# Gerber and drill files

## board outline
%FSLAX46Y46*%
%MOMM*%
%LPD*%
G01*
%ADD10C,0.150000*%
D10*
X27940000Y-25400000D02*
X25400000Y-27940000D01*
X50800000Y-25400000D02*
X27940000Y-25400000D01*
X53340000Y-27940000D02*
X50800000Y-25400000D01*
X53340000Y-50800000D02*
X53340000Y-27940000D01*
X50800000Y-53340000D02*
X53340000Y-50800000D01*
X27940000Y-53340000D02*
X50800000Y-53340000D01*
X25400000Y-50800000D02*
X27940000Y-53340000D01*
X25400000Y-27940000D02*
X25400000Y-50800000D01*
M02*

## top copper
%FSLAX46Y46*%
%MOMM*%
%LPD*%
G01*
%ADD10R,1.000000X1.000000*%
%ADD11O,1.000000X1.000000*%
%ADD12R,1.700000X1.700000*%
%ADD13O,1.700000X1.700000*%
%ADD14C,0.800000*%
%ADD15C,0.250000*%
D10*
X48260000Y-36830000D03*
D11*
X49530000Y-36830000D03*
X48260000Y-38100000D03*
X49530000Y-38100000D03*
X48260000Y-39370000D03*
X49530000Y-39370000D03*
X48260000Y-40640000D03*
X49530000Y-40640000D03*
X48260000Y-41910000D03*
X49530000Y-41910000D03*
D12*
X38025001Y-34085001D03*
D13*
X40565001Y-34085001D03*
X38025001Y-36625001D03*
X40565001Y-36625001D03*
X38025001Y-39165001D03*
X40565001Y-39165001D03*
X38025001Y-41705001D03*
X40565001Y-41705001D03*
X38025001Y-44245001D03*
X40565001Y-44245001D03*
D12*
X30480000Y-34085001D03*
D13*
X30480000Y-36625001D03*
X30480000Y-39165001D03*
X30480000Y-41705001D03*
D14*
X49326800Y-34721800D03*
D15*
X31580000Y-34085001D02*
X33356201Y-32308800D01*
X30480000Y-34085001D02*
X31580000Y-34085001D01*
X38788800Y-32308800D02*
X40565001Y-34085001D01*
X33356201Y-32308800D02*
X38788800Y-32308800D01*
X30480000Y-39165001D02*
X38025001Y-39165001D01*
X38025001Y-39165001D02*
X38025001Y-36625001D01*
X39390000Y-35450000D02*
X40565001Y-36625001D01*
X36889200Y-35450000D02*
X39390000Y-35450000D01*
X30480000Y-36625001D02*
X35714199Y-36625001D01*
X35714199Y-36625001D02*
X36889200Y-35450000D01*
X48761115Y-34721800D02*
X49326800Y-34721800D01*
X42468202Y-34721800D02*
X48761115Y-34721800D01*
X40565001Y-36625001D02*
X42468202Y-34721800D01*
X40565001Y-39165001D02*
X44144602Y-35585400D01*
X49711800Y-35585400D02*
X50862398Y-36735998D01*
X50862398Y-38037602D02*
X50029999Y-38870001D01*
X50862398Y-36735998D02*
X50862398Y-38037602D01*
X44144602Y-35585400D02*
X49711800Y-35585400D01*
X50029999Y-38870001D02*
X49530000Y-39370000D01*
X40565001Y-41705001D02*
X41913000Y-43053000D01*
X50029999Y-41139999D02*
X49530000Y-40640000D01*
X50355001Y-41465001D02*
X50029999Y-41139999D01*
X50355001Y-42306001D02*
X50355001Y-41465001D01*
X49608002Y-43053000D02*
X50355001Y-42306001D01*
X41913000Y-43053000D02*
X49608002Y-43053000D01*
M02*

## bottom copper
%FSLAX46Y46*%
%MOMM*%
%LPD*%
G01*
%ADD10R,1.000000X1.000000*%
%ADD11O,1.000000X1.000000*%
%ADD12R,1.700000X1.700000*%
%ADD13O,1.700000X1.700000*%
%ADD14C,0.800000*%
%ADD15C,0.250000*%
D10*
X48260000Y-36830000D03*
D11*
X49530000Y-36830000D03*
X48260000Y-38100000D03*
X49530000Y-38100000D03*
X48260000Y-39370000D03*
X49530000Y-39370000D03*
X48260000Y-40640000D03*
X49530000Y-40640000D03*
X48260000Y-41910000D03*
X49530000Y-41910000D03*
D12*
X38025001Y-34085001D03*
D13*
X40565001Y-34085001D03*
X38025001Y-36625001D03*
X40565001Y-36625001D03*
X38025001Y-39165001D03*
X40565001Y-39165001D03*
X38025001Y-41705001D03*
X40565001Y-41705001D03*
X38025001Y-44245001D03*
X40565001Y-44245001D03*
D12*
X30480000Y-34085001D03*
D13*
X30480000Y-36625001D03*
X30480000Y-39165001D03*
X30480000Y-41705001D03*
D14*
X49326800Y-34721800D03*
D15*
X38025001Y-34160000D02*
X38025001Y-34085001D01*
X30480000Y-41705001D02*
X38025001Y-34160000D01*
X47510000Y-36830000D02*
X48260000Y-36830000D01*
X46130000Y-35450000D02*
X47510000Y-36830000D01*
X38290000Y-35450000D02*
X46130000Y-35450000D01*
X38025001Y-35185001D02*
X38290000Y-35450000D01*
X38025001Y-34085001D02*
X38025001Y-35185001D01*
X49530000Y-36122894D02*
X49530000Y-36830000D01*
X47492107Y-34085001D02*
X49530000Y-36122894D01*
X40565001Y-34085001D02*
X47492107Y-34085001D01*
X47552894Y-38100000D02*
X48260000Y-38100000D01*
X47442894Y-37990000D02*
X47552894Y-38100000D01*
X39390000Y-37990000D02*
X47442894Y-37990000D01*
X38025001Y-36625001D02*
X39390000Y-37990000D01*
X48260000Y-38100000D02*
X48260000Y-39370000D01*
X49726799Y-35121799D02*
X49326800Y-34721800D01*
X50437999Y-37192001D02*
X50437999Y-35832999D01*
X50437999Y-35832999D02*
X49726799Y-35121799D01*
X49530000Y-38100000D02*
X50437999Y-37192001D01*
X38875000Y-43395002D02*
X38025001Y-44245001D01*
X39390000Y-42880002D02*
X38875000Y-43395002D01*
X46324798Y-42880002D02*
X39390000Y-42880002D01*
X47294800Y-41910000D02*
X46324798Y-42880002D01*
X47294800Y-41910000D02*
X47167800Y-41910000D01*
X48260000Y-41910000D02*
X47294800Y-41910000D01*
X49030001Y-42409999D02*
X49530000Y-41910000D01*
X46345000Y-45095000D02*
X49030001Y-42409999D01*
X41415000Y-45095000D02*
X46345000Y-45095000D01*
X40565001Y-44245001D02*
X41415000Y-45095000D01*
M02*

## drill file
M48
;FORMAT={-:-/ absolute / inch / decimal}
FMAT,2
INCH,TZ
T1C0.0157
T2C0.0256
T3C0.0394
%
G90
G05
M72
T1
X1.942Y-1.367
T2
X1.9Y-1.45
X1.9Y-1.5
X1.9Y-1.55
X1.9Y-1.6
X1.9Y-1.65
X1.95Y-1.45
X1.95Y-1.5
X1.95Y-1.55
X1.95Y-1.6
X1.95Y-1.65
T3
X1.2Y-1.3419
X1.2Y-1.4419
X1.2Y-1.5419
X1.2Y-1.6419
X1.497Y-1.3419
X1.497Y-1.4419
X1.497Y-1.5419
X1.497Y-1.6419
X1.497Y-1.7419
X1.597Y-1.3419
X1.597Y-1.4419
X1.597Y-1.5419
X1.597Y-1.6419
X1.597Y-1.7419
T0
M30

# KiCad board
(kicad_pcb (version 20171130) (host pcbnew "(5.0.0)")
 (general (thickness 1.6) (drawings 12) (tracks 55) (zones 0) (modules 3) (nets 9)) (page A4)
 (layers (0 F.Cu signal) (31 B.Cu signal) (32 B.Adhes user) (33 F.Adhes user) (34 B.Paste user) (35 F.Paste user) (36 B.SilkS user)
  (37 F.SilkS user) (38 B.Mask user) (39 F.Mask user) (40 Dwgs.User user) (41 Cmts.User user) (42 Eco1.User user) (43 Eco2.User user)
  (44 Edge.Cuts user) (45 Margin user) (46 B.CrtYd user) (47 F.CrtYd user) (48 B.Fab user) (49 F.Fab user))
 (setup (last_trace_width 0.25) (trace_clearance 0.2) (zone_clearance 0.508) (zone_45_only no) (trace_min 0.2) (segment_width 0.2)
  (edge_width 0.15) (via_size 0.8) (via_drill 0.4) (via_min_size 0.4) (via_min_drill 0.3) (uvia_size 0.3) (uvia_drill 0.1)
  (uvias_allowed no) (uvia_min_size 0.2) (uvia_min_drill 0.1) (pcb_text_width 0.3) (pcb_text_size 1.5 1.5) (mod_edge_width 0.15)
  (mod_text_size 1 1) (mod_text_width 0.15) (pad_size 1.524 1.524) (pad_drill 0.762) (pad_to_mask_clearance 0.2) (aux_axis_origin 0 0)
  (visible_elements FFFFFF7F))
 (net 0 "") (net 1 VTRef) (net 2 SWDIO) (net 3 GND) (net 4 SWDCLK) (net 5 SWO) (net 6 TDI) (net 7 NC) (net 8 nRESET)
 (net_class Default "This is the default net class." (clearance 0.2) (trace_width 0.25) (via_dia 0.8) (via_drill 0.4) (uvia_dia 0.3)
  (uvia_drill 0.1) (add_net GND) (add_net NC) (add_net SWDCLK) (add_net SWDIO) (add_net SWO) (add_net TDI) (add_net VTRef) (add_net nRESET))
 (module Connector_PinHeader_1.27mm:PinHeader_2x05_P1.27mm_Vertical (layer F.Cu) (at 48.26 36.83)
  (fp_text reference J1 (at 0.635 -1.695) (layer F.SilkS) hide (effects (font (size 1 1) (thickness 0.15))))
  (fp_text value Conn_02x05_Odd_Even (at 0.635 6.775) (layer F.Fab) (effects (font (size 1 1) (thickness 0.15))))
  (pad 1 thru_hole rect (at 0 0) (size 1 1) (drill 0.65) (layers *.Cu *.Mask) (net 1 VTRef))
  (pad 2 thru_hole oval (at 1.27 0) (size 1 1) (drill 0.65) (layers *.Cu *.Mask) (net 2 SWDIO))
  (pad 3 thru_hole oval (at 0 1.27) (size 1 1) (drill 0.65) (layers *.Cu *.Mask) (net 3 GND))
  (pad 4 thru_hole oval (at 1.27 1.27) (size 1 1) (drill 0.65) (layers *.Cu *.Mask) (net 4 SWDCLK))
  (pad 5 thru_hole oval (at 0 2.54) (size 1 1) (drill 0.65) (layers *.Cu *.Mask) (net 3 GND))
  (pad 6 thru_hole oval (at 1.27 2.54) (size 1 1) (drill 0.65) (layers *.Cu *.Mask) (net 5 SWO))
  (pad 7 thru_hole oval (at 0 3.81) (size 1 1) (drill 0.65) (layers *.Cu *.Mask))
  (pad 8 thru_hole oval (at 1.27 3.81) (size 1 1) (drill 0.65) (layers *.Cu *.Mask) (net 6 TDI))
  (pad 9 thru_hole oval (at 0 5.08) (size 1 1) (drill 0.65) (layers *.Cu *.Mask) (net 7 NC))
  (pad 10 thru_hole oval (at 1.27 5.08) (size 1 1) (drill 0.65) (layers *.Cu *.Mask) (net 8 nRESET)))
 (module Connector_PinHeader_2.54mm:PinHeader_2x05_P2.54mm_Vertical (layer F.Cu) (at 38.025001 34.085001)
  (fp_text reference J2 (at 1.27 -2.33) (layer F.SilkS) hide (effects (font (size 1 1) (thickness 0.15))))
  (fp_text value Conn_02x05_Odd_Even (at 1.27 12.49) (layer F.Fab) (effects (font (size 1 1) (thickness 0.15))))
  (pad 1 thru_hole rect (at 0 0) (size 1.7 1.7) (drill 1) (layers *.Cu *.Mask) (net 1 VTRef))
  (pad 2 thru_hole oval (at 2.54 0) (size 1.7 1.7) (drill 1) (layers *.Cu *.Mask) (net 2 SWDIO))
  (pad 3 thru_hole oval (at 0 2.54) (size 1.7 1.7) (drill 1) (layers *.Cu *.Mask) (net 3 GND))
  (pad 4 thru_hole oval (at 2.54 2.54) (size 1.7 1.7) (drill 1) (layers *.Cu *.Mask) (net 4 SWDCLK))
  (pad 5 thru_hole oval (at 0 5.08) (size 1.7 1.7) (drill 1) (layers *.Cu *.Mask) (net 3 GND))
  (pad 6 thru_hole oval (at 2.54 5.08) (size 1.7 1.7) (drill 1) (layers *.Cu *.Mask) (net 5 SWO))
  (pad 7 thru_hole oval (at 0 7.62) (size 1.7 1.7) (drill 1) (layers *.Cu *.Mask))
  (pad 8 thru_hole oval (at 2.54 7.62) (size 1.7 1.7) (drill 1) (layers *.Cu *.Mask) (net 6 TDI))
  (pad 9 thru_hole oval (at 0 10.16) (size 1.7 1.7) (drill 1) (layers *.Cu *.Mask) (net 7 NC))
  (pad 10 thru_hole oval (at 2.54 10.16) (size 1.7 1.7) (drill 1) (layers *.Cu *.Mask) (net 8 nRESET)))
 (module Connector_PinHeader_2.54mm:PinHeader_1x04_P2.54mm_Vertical (layer F.Cu) (at 30.48 34.085001)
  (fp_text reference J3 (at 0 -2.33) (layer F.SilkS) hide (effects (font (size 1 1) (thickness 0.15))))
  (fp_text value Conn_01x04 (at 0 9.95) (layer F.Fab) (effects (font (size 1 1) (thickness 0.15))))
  (pad 1 thru_hole rect (at 0 0) (size 1.7 1.7) (drill 1) (layers *.Cu *.Mask) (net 2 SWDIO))
  (pad 2 thru_hole oval (at 0 2.54) (size 1.7 1.7) (drill 1) (layers *.Cu *.Mask) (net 4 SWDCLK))
  (pad 3 thru_hole oval (at 0 5.08) (size 1.7 1.7) (drill 1) (layers *.Cu *.Mask) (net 3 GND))
  (pad 4 thru_hole oval (at 0 7.62) (size 1.7 1.7) (drill 1) (layers *.Cu *.Mask) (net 1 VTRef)))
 (gr_line (start 27.94 25.4) (end 25.4 27.94) (layer Edge.Cuts) (width 0.15))
 (gr_line (start 50.8 25.4) (end 27.94 25.4) (layer Edge.Cuts) (width 0.15))
 (gr_line (start 53.34 27.94) (end 50.8 25.4) (layer Edge.Cuts) (width 0.15))
 (gr_line (start 53.34 50.8) (end 53.34 27.94) (layer Edge.Cuts) (width 0.15))
 (gr_line (start 50.8 53.34) (end 53.34 50.8) (layer Edge.Cuts) (width 0.15))
 (gr_line (start 27.94 53.34) (end 50.8 53.34) (layer Edge.Cuts) (width 0.15))
 (gr_line (start 25.4 50.8) (end 27.94 53.34) (layer Edge.Cuts) (width 0.15))
 (gr_line (start 25.4 27.94) (end 25.4 50.8) (layer Edge.Cuts) (width 0.15))
 (segment (start 38.025001 34.16) (end 38.025001 34.085001) (width 0.25) (layer B.Cu) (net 1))
 (segment (start 30.48 41.705001) (end 38.025001 34.16) (width 0.25) (layer B.Cu) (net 1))
 (segment (start 47.51 36.83) (end 48.26 36.83) (width 0.25) (layer B.Cu) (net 1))
 (segment (start 46.13 35.45) (end 47.51 36.83) (width 0.25) (layer B.Cu) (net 1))
 (segment (start 38.29 35.45) (end 46.13 35.45) (width 0.25) (layer B.Cu) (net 1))
 (segment (start 38.025001 35.185001) (end 38.29 35.45) (width 0.25) (layer B.Cu) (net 1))
 (segment (start 38.025001 34.085001) (end 38.025001 35.185001) (width 0.25) (layer B.Cu) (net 1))
 (segment (start 31.58 34.085001) (end 33.356201 32.3088) (width 0.25) (layer F.Cu) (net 2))
 (segment (start 30.48 34.085001) (end 31.58 34.085001) (width 0.25) (layer F.Cu) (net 2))
 (segment (start 38.7888 32.3088) (end 40.565001 34.085001) (width 0.25) (layer F.Cu) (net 2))
 (segment (start 33.356201 32.3088) (end 38.7888 32.3088) (width 0.25) (layer F.Cu) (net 2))
 (segment (start 49.53 36.122894) (end 49.53 36.83) (width 0.25) (layer B.Cu) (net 2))
 (segment (start 47.492107 34.085001) (end 49.53 36.122894) (width 0.25) (layer B.Cu) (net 2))
 (segment (start 40.565001 34.085001) (end 47.492107 34.085001) (width 0.25) (layer B.Cu) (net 2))
 (segment (start 30.48 39.165001) (end 38.025001 39.165001) (width 0.25) (layer F.Cu) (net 3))
 (segment (start 38.025001 39.165001) (end 38.025001 36.625001) (width 0.25) (layer F.Cu) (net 3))
 (segment (start 47.552894 38.1) (end 48.26 38.1) (width 0.25) (layer B.Cu) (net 3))
 (segment (start 47.442894 37.99) (end 47.552894 38.1) (width 0.25) (layer B.Cu) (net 3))
 (segment (start 39.39 37.99) (end 47.442894 37.99) (width 0.25) (layer B.Cu) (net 3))
 (segment (start 38.025001 36.625001) (end 39.39 37.99) (width 0.25) (layer B.Cu) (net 3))
 (segment (start 48.26 38.1) (end 48.26 39.37) (width 0.25) (layer B.Cu) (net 3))
 (segment (start 39.39 35.45) (end 40.565001 36.625001) (width 0.25) (layer F.Cu) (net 4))
 (segment (start 36.8892 35.45) (end 39.39 35.45) (width 0.25) (layer F.Cu) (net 4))
 (segment (start 30.48 36.625001) (end 35.714199 36.625001) (width 0.25) (layer F.Cu) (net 4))
 (segment (start 35.714199 36.625001) (end 36.8892 35.45) (width 0.25) (layer F.Cu) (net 4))
 (segment (start 49.726799 35.121799) (end 49.3268 34.7218) (width 0.25) (layer B.Cu) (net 4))
 (segment (start 48.761115 34.7218) (end 49.3268 34.7218) (width 0.25) (layer F.Cu) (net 4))
 (segment (start 50.437999 37.192001) (end 50.437999 35.832999) (width 0.25) (layer B.Cu) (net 4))
 (segment (start 50.437999 35.832999) (end 49.726799 35.121799) (width 0.25) (layer B.Cu) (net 4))
 (segment (start 49.53 38.1) (end 50.437999 37.192001) (width 0.25) (layer B.Cu) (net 4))
 (segment (start 42.468202 34.7218) (end 48.761115 34.7218) (width 0.25) (layer F.Cu) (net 4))
 (segment (start 40.565001 36.625001) (end 42.468202 34.7218) (width 0.25) (layer F.Cu) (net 4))
 (via (at 49.3268 34.7218) (size 0.8) (drill 0.4) (layers F.Cu B.Cu) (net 4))
 (segment (start 40.565001 39.165001) (end 44.144602 35.5854) (width 0.25) (layer F.Cu) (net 5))
 (segment (start 49.7118 35.5854) (end 50.862398 36.735998) (width 0.25) (layer F.Cu) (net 5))
 (segment (start 50.862398 38.037602) (end 50.029999 38.870001) (width 0.25) (layer F.Cu) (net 5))
 (segment (start 50.862398 36.735998) (end 50.862398 38.037602) (width 0.25) (layer F.Cu) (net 5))
 (segment (start 44.144602 35.5854) (end 49.7118 35.5854) (width 0.25) (layer F.Cu) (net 5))
 (segment (start 50.029999 38.870001) (end 49.53 39.37) (width 0.25) (layer F.Cu) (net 5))
 (segment (start 40.565001 41.705001) (end 41.913 43.053) (width 0.25) (layer F.Cu) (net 6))
 (segment (start 50.029999 41.139999) (end 49.53 40.64) (width 0.25) (layer F.Cu) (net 6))
 (segment (start 50.355001 41.465001) (end 50.029999 41.139999) (width 0.25) (layer F.Cu) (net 6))
 (segment (start 50.355001 42.306001) (end 50.355001 41.465001) (width 0.25) (layer F.Cu) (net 6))
 (segment (start 49.608002 43.053) (end 50.355001 42.306001) (width 0.25) (layer F.Cu) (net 6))
 (segment (start 41.913 43.053) (end 49.608002 43.053) (width 0.25) (layer F.Cu) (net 6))
 (segment (start 38.875 43.395002) (end 38.025001 44.245001) (width 0.25) (layer B.Cu) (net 7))
 (segment (start 39.39 42.880002) (end 38.875 43.395002) (width 0.25) (layer B.Cu) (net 7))
 (segment (start 46.324798 42.880002) (end 39.39 42.880002) (width 0.25) (layer B.Cu) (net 7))
 (segment (start 47.2948 41.91) (end 46.324798 42.880002) (width 0.25) (layer B.Cu) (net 7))
 (segment (start 47.2948 41.91) (end 47.1678 41.91) (width 0.25) (layer B.Cu) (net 7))
 (segment (start 48.26 41.91) (end 47.2948 41.91) (width 0.25) (layer B.Cu) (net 7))
 (segment (start 49.030001 42.409999) (end 49.53 41.91) (width 0.25) (layer B.Cu) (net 8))
 (segment (start 46.345 45.095) (end 49.030001 42.409999) (width 0.25) (layer B.Cu) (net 8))
 (segment (start 41.415 45.095) (end 46.345 45.095) (width 0.25) (layer B.Cu) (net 8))
 (segment (start 40.565001 44.245001) (end 41.415 45.095) (width 0.25) (layer B.Cu) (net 8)))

